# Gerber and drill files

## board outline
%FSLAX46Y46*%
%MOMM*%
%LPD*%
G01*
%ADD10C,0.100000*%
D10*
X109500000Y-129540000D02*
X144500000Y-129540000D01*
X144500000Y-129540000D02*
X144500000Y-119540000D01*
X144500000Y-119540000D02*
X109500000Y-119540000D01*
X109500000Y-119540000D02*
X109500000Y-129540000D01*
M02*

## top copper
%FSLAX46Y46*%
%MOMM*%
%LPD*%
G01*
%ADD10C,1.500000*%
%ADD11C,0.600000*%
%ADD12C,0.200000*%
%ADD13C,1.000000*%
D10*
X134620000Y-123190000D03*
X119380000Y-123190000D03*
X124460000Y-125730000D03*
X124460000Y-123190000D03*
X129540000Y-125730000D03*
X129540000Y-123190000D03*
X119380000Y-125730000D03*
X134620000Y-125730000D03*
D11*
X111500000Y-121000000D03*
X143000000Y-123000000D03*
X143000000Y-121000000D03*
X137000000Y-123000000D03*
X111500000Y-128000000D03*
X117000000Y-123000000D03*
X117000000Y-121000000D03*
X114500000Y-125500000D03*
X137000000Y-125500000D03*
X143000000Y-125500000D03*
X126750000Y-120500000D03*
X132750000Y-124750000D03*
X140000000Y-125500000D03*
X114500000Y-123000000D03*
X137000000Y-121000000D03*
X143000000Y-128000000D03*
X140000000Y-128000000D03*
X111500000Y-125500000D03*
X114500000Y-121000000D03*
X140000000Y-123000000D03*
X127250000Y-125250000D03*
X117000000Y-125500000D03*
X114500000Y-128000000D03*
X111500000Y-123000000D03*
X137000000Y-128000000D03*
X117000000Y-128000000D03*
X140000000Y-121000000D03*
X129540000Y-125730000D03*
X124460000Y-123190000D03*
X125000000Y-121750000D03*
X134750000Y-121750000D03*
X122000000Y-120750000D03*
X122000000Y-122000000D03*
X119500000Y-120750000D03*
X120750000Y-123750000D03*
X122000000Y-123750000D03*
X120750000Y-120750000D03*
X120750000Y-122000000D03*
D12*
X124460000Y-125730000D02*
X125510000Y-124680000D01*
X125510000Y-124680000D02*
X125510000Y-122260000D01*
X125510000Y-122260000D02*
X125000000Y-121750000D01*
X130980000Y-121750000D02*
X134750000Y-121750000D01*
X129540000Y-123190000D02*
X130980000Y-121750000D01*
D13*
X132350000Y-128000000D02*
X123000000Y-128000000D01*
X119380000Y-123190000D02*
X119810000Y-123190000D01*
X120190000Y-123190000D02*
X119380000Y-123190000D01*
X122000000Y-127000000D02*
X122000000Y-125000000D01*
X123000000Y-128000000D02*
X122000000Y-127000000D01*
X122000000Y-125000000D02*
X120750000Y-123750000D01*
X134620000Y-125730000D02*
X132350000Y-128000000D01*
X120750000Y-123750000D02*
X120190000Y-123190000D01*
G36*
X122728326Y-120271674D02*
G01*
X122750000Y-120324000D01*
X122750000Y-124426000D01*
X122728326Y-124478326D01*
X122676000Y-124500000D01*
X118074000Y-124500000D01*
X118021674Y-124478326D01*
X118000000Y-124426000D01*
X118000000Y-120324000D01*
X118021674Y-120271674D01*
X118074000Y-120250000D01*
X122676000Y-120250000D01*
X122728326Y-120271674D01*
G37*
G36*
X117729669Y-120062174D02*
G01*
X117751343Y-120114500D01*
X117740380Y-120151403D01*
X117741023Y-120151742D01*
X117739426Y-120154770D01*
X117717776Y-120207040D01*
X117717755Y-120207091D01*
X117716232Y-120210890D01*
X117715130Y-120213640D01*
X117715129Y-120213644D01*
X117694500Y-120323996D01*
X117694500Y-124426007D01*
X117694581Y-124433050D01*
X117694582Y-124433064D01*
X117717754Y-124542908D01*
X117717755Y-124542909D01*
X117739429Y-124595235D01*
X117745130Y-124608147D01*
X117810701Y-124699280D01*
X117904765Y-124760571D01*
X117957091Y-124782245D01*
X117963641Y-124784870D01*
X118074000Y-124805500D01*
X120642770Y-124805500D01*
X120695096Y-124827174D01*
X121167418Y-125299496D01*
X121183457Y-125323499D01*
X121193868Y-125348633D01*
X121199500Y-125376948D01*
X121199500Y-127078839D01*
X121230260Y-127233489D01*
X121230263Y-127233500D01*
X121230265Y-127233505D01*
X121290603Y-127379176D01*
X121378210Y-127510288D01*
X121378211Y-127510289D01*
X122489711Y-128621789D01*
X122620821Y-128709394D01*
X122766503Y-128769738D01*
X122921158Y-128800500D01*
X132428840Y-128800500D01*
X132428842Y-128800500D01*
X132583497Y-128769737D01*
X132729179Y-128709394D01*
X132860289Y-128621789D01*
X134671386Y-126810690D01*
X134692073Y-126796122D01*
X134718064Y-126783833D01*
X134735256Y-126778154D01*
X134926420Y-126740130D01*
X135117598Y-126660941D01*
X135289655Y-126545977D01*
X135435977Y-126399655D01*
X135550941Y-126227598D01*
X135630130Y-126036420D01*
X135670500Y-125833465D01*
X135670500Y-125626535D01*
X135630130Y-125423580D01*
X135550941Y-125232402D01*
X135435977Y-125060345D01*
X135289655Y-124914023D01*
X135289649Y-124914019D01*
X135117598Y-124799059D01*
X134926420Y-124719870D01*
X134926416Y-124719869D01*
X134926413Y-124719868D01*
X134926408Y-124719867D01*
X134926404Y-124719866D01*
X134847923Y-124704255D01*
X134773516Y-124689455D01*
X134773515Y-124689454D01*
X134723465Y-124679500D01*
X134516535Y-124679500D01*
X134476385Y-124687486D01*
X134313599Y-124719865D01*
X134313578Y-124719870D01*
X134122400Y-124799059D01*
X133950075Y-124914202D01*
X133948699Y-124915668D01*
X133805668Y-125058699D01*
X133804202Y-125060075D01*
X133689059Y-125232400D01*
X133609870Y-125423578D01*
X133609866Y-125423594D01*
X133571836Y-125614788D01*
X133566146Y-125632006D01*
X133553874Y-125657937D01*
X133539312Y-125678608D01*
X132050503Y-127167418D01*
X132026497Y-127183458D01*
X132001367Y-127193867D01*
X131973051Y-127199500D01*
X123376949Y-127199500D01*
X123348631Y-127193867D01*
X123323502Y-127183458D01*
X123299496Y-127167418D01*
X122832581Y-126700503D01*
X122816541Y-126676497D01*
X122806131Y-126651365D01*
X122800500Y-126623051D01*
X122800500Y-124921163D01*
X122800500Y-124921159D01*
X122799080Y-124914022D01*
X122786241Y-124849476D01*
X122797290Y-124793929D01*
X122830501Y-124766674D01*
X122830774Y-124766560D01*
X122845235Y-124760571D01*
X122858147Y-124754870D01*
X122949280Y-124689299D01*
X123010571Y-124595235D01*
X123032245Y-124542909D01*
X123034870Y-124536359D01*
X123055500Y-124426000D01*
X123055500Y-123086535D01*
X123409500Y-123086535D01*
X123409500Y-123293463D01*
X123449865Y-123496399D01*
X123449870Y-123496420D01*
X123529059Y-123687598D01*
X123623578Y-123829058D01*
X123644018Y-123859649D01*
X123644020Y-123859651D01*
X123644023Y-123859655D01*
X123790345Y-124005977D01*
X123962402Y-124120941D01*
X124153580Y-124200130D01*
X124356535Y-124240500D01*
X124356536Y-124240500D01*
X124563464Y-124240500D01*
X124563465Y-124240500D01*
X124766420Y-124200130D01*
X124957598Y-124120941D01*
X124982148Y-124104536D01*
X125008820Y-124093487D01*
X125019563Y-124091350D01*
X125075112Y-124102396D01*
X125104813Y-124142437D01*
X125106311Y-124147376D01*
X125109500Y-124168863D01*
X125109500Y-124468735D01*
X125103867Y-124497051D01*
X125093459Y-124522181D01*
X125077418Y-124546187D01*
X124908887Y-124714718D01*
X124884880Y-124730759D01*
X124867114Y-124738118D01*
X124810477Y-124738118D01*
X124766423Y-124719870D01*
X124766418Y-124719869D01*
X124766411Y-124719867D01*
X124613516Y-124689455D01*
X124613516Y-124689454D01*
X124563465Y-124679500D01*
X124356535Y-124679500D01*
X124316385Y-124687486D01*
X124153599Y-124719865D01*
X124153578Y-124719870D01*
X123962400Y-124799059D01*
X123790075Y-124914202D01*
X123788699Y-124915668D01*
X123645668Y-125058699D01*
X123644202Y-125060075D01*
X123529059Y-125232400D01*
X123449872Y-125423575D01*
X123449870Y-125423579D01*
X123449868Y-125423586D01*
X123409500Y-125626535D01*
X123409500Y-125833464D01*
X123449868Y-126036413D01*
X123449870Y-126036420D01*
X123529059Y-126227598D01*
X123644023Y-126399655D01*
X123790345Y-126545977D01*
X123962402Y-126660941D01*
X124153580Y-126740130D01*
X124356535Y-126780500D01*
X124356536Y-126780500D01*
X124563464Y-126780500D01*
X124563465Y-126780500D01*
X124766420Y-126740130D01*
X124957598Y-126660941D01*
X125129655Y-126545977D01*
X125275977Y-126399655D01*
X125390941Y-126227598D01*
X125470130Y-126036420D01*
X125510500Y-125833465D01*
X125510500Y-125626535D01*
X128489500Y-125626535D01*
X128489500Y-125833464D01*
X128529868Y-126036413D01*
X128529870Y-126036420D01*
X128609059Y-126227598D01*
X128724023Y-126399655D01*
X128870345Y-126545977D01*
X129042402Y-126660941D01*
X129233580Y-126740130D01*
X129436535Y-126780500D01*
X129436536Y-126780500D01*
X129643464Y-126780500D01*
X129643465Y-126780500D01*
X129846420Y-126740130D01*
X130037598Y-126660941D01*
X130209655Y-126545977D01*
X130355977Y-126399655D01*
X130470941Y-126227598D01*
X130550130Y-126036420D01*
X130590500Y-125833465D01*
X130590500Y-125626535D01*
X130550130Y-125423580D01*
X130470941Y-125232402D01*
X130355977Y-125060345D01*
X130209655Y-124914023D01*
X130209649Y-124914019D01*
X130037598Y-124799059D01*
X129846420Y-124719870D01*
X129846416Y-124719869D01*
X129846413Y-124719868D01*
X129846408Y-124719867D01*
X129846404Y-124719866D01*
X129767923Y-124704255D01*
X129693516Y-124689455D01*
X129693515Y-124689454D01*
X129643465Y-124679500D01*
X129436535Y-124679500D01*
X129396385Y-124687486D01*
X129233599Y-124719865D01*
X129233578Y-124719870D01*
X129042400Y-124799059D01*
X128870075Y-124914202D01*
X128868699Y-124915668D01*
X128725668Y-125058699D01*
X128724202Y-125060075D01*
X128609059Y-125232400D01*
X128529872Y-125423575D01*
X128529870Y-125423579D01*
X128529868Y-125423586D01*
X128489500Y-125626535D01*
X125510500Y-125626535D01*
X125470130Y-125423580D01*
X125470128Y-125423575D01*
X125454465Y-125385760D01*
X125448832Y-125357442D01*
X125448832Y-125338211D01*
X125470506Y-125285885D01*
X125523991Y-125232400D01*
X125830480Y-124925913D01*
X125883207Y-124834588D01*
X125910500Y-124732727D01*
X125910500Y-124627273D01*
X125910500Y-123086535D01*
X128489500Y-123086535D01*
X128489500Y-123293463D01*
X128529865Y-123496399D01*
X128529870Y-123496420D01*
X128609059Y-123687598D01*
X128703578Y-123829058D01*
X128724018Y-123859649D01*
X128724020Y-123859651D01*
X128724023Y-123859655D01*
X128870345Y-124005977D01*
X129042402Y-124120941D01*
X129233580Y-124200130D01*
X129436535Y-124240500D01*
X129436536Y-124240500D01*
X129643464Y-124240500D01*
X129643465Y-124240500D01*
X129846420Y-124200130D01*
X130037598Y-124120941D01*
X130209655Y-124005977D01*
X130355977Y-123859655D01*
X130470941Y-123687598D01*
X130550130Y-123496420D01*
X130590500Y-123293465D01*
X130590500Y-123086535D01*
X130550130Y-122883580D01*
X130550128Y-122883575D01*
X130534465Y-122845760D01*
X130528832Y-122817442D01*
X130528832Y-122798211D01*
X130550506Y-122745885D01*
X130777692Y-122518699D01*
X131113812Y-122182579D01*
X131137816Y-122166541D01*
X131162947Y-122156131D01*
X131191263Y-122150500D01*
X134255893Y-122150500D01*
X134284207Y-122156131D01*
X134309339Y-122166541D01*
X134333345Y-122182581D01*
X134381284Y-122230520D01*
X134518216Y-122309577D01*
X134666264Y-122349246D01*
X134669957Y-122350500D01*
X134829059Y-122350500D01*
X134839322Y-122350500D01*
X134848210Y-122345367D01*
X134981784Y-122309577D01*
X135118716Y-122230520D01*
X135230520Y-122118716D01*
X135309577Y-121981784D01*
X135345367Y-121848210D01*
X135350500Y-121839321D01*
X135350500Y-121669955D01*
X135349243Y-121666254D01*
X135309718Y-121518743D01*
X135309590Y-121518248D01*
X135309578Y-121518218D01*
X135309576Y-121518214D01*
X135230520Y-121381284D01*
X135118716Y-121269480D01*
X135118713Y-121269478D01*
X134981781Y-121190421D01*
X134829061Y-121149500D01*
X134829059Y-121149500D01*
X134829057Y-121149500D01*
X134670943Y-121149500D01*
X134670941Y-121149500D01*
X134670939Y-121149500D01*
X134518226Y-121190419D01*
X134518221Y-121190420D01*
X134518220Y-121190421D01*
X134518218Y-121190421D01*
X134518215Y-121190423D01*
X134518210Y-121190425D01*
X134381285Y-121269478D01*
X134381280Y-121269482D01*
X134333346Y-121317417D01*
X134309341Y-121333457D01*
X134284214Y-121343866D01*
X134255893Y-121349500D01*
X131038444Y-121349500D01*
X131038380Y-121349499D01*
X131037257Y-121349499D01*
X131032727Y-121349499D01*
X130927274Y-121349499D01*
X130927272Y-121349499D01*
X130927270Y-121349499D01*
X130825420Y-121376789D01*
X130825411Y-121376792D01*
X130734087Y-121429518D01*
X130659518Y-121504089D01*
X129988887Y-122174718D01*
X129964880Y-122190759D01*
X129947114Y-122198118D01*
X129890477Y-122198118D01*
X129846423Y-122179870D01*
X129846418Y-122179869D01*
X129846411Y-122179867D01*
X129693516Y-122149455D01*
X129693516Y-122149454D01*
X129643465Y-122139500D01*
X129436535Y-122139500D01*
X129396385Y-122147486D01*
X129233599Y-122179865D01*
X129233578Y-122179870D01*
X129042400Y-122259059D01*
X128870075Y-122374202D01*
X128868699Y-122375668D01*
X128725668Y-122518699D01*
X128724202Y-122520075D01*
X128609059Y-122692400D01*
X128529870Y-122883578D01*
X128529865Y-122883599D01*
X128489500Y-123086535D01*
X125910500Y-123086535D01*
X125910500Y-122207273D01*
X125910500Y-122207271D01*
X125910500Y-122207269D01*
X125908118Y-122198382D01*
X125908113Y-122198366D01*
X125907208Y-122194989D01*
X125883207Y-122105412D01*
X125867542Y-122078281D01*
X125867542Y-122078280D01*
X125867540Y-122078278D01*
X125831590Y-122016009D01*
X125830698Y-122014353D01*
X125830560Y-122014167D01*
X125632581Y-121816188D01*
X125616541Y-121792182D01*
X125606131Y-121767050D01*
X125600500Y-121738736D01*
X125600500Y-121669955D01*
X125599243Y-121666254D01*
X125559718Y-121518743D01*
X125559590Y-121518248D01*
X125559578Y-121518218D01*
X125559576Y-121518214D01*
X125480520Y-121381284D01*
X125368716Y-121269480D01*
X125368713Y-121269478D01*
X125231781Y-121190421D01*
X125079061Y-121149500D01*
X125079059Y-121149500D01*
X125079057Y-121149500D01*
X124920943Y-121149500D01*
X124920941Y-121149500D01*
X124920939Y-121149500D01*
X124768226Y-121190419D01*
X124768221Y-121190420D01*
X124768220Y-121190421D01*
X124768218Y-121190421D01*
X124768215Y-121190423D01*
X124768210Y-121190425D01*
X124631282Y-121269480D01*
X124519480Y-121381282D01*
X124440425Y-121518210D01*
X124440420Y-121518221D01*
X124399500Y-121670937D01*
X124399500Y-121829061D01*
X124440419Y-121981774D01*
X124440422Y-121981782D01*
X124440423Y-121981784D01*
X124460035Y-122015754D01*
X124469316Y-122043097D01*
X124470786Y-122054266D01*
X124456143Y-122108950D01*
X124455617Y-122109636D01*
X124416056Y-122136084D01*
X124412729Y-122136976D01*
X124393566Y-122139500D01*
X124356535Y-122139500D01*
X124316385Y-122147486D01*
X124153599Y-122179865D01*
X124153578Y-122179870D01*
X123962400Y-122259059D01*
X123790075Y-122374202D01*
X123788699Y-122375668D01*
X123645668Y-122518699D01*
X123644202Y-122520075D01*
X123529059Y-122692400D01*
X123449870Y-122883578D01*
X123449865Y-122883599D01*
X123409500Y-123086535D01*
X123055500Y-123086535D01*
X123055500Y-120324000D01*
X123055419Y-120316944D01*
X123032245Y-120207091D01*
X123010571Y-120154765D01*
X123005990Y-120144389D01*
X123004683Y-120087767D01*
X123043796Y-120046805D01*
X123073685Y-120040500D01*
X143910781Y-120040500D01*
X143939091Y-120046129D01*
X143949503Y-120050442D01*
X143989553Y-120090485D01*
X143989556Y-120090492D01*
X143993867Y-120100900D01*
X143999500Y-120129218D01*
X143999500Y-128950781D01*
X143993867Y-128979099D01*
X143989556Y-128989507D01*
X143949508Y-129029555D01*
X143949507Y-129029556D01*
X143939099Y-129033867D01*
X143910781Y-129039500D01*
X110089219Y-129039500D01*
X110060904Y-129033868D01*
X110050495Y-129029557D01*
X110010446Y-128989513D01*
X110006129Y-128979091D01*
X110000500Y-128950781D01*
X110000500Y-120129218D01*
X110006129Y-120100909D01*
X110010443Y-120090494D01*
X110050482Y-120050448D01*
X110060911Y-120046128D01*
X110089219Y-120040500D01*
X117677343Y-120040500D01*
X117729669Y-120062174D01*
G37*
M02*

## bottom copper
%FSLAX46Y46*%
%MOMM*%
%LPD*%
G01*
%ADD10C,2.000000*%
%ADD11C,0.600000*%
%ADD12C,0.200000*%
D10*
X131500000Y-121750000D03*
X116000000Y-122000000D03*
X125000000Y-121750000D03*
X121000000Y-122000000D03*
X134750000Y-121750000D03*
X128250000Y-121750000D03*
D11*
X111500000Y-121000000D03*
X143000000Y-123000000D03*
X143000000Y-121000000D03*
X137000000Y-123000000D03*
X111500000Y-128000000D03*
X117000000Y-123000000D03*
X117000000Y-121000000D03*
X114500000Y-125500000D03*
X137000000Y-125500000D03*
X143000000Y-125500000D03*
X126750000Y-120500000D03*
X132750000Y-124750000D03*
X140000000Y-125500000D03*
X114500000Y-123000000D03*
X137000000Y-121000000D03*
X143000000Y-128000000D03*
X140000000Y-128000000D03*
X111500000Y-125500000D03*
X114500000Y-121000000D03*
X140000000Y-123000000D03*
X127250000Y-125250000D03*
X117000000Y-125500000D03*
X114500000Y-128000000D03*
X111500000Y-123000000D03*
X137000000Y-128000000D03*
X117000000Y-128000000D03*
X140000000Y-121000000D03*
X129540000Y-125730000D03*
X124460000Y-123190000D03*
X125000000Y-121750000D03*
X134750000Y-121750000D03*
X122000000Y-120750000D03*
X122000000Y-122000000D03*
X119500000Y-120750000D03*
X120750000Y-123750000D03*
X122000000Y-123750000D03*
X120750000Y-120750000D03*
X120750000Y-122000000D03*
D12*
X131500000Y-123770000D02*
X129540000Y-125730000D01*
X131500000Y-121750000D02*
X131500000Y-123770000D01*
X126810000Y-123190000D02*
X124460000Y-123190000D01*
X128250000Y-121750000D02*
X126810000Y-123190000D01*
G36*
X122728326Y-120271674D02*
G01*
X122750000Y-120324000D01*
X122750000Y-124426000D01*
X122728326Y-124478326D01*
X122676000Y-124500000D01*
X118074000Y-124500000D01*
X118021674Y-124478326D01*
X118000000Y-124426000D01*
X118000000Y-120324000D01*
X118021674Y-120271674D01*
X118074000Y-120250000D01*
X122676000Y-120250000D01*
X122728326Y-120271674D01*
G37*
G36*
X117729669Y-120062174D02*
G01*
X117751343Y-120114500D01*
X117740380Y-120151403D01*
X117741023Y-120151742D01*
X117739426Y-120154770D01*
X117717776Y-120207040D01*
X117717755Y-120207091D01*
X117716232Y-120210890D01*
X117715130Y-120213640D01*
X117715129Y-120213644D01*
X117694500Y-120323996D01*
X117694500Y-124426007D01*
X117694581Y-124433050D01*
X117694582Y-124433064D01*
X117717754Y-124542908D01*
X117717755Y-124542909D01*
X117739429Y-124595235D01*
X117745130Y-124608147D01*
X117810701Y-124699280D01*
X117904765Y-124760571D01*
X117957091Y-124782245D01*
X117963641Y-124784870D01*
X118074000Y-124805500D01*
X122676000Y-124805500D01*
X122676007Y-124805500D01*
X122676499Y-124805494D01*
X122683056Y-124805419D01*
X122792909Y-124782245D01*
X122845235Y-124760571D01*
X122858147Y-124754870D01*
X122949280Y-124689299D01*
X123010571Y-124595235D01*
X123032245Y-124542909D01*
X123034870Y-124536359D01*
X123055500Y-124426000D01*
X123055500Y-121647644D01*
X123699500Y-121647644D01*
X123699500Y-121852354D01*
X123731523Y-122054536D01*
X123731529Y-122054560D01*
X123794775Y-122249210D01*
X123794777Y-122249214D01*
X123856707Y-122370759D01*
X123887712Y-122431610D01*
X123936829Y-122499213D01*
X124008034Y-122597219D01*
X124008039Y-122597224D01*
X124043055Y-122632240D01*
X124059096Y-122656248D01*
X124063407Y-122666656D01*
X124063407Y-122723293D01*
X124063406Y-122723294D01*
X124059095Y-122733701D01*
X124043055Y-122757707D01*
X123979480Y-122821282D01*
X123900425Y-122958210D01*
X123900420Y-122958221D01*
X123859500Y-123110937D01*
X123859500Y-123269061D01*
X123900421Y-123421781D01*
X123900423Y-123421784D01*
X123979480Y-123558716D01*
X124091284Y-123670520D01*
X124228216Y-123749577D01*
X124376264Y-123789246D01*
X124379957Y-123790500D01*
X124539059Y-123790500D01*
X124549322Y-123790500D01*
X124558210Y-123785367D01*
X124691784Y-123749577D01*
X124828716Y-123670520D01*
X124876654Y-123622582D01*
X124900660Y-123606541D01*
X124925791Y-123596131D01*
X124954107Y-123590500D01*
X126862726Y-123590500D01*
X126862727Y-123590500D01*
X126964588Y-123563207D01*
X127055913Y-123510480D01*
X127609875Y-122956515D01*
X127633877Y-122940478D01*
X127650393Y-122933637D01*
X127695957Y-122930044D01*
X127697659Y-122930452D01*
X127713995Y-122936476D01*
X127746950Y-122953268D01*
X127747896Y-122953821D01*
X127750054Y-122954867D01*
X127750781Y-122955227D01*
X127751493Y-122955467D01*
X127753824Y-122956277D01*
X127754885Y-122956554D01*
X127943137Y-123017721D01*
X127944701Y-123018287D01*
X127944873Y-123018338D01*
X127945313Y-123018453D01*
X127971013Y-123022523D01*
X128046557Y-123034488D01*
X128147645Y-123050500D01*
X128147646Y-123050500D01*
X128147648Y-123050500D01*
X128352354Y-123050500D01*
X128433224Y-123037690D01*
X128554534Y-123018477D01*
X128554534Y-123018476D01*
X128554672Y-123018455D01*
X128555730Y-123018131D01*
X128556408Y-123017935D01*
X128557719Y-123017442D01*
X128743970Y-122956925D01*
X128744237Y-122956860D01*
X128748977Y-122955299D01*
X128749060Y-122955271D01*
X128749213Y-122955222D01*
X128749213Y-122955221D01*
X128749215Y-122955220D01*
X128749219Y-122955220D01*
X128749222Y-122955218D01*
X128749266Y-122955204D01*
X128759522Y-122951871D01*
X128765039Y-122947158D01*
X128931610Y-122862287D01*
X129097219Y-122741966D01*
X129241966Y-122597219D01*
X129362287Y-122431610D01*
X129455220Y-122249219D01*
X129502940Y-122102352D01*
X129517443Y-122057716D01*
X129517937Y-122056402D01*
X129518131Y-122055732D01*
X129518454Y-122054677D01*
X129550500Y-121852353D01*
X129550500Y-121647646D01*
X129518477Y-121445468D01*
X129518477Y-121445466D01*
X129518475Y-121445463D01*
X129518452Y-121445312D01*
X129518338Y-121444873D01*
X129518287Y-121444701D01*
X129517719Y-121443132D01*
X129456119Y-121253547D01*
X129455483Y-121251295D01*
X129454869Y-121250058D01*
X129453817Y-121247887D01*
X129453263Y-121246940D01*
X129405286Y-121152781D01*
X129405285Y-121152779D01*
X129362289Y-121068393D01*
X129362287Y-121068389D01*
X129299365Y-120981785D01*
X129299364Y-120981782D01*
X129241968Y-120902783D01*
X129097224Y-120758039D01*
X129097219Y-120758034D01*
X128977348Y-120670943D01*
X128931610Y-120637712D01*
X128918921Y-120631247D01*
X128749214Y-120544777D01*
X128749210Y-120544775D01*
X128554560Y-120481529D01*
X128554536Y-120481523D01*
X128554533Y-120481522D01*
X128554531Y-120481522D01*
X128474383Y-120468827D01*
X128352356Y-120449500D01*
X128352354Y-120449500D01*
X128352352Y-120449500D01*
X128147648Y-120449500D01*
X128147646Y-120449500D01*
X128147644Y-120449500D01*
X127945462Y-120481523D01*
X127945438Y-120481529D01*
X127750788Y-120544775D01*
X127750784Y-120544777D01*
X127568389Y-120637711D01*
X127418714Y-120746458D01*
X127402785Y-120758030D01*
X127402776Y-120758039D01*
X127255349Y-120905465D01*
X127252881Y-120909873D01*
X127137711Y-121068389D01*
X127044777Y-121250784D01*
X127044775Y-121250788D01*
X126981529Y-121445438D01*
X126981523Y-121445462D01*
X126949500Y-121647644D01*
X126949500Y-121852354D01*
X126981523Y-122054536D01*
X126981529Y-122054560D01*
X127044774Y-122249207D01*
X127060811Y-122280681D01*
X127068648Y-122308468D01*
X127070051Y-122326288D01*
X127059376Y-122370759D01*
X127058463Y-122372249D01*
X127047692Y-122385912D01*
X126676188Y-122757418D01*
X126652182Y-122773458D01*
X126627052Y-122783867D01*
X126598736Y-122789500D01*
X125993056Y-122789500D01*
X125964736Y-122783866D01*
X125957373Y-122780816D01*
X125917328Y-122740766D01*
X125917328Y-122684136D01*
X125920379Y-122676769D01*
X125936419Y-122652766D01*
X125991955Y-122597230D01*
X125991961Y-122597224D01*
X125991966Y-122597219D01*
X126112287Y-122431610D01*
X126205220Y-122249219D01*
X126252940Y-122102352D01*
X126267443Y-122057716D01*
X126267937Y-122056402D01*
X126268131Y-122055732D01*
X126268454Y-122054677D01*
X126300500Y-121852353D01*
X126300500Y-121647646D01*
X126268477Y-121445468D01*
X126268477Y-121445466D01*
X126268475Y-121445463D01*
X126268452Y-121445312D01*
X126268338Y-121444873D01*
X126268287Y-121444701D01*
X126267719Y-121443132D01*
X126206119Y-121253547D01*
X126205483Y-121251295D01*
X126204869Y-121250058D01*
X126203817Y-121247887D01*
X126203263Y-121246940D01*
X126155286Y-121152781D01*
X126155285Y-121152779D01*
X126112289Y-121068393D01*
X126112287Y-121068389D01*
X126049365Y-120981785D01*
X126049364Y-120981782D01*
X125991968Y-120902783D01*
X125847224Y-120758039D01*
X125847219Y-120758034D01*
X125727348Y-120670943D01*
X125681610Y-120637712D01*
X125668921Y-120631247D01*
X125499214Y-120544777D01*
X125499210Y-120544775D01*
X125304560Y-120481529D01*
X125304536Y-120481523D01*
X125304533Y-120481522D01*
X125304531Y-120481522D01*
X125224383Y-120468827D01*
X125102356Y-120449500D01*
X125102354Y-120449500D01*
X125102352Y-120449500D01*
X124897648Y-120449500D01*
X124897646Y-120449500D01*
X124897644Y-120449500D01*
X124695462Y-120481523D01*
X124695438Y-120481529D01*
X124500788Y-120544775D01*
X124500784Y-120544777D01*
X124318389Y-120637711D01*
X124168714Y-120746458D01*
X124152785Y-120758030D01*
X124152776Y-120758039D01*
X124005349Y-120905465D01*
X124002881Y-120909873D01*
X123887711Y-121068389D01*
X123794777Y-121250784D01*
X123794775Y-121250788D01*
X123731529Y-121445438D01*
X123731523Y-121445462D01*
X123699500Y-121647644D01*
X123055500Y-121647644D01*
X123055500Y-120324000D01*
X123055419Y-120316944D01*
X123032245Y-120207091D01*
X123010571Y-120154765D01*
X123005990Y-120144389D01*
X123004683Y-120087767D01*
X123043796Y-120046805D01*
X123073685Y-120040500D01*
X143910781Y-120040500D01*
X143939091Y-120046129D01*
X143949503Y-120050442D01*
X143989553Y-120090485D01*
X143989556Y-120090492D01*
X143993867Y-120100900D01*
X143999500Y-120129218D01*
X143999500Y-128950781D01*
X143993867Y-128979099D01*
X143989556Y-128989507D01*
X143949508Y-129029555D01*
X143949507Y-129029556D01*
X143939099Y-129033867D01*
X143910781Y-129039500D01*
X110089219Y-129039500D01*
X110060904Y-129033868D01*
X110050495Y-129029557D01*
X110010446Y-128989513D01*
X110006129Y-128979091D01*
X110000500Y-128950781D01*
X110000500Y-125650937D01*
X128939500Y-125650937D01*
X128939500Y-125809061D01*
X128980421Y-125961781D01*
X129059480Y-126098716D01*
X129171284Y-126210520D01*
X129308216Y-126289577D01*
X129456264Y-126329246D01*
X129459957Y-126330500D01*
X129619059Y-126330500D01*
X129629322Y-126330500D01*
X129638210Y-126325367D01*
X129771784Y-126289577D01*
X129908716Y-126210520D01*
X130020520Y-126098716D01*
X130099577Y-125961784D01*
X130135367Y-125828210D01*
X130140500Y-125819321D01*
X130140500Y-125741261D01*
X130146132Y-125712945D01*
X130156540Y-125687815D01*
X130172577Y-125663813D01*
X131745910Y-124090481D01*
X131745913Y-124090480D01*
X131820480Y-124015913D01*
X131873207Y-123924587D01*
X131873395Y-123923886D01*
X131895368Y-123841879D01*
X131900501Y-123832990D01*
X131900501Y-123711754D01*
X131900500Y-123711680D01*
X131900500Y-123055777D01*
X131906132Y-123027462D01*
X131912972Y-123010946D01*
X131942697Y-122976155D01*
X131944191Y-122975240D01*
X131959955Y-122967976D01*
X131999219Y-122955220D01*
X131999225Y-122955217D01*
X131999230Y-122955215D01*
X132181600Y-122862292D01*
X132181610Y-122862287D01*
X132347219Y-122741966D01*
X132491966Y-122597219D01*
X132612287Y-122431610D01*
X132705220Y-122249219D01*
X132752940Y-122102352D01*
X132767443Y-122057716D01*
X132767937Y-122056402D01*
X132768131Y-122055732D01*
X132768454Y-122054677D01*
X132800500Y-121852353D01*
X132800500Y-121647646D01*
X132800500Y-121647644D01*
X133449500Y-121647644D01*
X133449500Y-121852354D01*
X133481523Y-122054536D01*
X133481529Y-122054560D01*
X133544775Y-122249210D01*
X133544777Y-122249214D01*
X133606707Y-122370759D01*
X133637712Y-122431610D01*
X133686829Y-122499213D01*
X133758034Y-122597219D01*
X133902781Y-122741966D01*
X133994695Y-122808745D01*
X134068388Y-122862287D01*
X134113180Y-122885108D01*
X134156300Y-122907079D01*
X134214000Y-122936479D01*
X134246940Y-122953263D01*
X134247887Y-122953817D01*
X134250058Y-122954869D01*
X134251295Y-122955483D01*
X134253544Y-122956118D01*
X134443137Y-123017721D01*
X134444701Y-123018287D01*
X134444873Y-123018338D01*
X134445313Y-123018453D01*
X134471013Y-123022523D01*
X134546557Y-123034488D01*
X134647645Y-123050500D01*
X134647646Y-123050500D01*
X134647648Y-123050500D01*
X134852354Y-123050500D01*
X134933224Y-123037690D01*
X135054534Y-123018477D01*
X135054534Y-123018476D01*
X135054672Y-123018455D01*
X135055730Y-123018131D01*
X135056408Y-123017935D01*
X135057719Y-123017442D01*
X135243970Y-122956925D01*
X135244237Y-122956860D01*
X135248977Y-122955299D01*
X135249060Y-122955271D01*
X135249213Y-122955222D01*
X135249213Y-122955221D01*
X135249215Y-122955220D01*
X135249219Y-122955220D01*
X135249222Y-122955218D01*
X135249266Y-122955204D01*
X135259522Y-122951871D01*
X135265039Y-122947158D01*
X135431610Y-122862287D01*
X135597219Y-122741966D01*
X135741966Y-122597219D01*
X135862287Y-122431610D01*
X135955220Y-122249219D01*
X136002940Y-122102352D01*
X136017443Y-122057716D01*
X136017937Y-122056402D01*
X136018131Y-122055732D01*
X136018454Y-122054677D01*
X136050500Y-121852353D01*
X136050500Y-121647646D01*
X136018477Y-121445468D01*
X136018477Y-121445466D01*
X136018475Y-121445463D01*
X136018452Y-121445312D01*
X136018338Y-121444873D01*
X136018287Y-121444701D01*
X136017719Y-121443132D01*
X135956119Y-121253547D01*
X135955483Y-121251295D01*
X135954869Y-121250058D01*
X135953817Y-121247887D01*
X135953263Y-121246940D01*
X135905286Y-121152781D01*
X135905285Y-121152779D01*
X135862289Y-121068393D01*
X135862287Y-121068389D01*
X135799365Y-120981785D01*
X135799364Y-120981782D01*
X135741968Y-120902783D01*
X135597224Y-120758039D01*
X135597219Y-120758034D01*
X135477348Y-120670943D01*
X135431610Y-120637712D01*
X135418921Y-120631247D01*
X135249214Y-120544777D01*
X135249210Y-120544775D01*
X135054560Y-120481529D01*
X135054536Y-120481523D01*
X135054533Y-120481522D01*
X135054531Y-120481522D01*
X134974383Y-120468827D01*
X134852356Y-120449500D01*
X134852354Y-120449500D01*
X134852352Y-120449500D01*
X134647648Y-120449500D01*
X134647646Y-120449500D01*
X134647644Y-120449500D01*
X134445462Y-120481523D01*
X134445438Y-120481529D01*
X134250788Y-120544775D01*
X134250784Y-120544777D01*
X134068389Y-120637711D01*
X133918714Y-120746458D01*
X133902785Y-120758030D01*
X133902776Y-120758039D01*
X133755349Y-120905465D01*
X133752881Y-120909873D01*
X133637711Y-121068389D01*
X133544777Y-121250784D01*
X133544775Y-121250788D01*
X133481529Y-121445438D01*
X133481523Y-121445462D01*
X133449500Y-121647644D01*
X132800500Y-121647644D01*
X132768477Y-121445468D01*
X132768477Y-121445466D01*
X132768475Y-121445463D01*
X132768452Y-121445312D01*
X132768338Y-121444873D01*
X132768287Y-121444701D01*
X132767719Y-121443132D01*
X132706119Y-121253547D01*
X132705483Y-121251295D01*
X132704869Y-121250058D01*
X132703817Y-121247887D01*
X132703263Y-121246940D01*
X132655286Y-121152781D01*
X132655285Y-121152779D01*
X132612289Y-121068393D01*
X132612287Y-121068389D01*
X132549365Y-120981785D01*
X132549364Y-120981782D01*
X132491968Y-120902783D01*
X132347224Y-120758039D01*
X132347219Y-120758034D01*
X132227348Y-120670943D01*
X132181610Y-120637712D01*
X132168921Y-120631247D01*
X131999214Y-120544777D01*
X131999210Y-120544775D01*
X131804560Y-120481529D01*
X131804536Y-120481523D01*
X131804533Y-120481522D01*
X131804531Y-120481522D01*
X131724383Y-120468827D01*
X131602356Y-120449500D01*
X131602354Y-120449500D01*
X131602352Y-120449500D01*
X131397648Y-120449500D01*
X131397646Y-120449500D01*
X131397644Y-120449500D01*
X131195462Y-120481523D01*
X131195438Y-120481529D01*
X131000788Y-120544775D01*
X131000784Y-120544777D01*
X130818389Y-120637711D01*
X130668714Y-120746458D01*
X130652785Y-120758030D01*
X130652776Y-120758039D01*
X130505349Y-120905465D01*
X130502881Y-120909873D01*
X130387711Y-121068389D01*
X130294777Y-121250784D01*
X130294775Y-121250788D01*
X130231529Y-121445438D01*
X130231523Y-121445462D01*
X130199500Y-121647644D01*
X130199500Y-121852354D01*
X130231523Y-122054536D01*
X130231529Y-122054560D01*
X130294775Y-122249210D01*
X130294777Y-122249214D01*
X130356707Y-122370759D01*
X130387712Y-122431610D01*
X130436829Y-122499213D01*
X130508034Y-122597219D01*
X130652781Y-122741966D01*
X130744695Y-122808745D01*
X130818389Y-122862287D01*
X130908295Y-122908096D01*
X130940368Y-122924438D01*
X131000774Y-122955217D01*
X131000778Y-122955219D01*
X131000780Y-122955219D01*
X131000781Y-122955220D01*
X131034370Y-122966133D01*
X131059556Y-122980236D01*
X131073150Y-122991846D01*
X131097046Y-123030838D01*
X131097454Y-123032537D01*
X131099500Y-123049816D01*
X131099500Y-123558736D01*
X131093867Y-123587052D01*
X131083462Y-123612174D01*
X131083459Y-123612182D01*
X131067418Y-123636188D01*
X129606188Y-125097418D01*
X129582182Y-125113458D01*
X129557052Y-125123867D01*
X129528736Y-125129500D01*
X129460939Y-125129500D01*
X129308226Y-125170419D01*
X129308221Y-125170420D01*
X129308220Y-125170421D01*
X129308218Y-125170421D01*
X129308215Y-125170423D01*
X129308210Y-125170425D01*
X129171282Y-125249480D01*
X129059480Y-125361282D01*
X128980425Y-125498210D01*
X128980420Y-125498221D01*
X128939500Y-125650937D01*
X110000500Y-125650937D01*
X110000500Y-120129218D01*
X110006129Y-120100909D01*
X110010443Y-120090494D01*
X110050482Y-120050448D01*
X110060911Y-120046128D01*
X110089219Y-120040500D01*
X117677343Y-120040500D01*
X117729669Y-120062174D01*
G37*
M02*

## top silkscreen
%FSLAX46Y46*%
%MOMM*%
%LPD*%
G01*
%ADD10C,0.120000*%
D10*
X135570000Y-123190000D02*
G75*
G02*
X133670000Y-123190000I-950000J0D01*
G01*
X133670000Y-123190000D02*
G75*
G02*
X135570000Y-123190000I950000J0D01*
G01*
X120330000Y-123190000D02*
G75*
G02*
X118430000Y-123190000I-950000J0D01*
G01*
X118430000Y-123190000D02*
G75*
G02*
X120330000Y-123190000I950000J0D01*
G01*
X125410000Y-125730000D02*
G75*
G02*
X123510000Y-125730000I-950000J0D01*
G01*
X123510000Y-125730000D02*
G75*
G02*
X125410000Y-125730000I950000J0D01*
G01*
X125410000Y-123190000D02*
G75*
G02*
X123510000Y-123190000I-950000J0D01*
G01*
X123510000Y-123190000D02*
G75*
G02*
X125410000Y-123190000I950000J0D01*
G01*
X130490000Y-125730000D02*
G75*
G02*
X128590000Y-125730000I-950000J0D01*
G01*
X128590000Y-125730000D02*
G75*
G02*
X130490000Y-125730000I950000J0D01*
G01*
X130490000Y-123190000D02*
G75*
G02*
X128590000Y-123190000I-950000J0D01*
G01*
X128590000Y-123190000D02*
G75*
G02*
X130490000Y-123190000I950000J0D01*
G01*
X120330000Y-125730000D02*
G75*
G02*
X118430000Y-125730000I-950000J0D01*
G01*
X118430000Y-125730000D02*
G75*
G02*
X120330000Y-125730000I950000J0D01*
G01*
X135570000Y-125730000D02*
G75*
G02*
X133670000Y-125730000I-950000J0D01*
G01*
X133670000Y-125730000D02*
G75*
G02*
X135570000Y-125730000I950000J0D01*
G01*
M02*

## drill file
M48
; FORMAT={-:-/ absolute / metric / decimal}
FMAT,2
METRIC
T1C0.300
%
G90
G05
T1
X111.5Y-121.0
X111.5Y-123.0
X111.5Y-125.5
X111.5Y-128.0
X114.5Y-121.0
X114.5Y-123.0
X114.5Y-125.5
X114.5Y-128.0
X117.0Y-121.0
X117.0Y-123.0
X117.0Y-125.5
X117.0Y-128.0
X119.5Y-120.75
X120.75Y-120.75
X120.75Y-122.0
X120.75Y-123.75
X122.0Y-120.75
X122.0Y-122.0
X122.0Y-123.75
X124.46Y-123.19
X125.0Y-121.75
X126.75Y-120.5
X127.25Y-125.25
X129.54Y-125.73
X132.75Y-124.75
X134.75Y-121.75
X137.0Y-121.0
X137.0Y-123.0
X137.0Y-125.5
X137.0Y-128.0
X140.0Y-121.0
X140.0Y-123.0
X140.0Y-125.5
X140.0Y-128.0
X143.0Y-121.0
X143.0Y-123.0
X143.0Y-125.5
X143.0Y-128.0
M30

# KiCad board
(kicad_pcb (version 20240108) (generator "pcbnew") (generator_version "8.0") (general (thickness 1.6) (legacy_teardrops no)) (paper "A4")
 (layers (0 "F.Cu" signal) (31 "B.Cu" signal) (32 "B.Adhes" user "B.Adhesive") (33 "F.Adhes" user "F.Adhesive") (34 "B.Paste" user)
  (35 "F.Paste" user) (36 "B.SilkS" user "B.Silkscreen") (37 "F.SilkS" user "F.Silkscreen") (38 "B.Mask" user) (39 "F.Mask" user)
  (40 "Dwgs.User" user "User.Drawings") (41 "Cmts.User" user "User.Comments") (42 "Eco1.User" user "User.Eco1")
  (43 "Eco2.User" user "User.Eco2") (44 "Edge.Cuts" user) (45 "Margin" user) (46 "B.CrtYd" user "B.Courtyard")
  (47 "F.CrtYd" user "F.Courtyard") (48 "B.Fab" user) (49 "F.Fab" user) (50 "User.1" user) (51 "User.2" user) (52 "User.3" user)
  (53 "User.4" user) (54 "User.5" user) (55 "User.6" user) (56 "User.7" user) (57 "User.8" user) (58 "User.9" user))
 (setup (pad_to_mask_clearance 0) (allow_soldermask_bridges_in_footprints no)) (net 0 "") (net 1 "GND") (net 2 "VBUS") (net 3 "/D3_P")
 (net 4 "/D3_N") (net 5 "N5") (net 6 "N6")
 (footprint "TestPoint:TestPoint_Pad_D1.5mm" (layer "F.Cu") (at 134.62 123.19)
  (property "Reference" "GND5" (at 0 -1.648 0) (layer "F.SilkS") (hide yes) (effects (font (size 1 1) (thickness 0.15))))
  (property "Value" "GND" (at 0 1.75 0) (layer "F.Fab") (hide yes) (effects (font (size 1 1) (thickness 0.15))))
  (fp_circle (center 0 0) (end 0 0.95) (stroke (width 0.12) (type solid)) (fill none) (layer "F.SilkS"))
  (pad "1" smd circle (at 0 0) (size 1.5 1.5) (layers "F.Cu" "F.Mask") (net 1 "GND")))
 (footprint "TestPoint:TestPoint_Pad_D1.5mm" (layer "F.Cu") (at 119.38 123.19)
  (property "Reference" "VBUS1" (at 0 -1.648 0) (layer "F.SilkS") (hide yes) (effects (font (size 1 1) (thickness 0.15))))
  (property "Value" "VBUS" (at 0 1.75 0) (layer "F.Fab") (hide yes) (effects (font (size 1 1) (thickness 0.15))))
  (fp_circle (center 0 0) (end 0 0.95) (stroke (width 0.12) (type solid)) (fill none) (layer "F.SilkS"))
  (pad "1" smd circle (at 0 0) (size 1.5 1.5) (layers "F.Cu" "F.Mask") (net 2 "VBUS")))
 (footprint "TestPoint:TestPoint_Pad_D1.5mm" (layer "F.Cu") (at 124.46 125.73 180)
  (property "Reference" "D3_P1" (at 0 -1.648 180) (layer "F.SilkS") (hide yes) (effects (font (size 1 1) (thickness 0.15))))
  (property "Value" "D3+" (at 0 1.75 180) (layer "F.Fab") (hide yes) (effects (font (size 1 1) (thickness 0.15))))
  (fp_circle (center 0 0) (end 0 0.95) (stroke (width 0.12) (type solid)) (fill none) (layer "F.SilkS"))
  (pad "1" smd circle (at 0 0 180) (size 1.5 1.5) (layers "F.Cu" "F.Mask") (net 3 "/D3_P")))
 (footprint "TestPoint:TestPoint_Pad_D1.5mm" (layer "F.Cu") (at 124.46 123.19)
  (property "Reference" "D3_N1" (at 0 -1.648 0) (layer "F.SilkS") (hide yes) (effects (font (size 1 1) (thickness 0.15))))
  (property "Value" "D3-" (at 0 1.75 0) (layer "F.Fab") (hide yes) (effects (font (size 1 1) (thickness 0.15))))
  (fp_circle (center 0 0) (end 0 0.95) (stroke (width 0.12) (type solid)) (fill none) (layer "F.SilkS"))
  (pad "1" smd circle (at 0 0) (size 1.5 1.5) (layers "F.Cu" "F.Mask") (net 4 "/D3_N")))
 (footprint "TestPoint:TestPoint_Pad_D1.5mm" (layer "F.Cu") (at 129.54 125.73 180)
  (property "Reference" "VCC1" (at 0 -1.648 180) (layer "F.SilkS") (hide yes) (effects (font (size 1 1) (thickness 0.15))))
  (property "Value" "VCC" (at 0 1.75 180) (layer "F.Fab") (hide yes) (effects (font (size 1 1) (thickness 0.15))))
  (fp_circle (center 0 0) (end 0 0.95) (stroke (width 0.12) (type solid)) (fill none) (layer "F.SilkS"))
  (pad "1" smd circle (at 0 0 180) (size 1.5 1.5) (layers "F.Cu" "F.Mask") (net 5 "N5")))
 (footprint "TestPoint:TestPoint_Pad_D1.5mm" (layer "F.Cu") (at 129.54 123.19)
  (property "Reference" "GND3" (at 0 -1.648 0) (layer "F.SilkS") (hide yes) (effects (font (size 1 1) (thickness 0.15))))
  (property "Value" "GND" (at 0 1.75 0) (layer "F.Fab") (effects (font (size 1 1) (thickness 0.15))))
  (fp_circle (center 0 0) (end 0 0.95) (stroke (width 0.12) (type solid)) (fill none) (layer "F.SilkS"))
  (pad "1" smd circle (at 0 0) (size 1.5 1.5) (layers "F.Cu" "F.Mask") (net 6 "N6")))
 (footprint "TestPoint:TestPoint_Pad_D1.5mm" (layer "F.Cu") (at 119.38 125.73 90)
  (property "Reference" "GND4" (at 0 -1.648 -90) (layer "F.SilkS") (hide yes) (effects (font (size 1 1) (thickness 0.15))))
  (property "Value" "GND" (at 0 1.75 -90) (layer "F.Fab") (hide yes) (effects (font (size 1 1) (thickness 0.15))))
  (fp_circle (center 0 0) (end 0 0.95) (stroke (width 0.12) (type solid)) (fill none) (layer "F.SilkS"))
  (pad "1" smd circle (at 0 0 90) (size 1.5 1.5) (layers "F.Cu" "F.Mask") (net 1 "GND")))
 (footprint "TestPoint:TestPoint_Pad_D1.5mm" (layer "F.Cu") (at 134.62 125.73)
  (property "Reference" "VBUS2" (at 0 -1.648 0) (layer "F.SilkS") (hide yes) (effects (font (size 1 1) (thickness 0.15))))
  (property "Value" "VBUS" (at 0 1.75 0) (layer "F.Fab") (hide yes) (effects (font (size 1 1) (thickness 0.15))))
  (fp_circle (center 0 0) (end 0 0.95) (stroke (width 0.12) (type solid)) (fill none) (layer "F.SilkS"))
  (pad "1" smd circle (at 0 0) (size 1.5 1.5) (layers "F.Cu" "F.Mask") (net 2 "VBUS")))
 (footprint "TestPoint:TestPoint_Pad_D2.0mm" (layer "B.Cu") (at 131.5 121.75 180)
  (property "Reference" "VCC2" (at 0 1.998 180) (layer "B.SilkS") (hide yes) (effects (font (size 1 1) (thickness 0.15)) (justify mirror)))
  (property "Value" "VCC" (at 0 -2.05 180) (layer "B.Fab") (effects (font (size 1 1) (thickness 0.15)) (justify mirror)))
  (pad "1" smd circle (at 0 0 180) (size 2 2) (layers "B.Cu" "B.Mask") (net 5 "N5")))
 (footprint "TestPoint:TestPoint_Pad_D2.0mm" (layer "B.Cu") (at 116 122 180)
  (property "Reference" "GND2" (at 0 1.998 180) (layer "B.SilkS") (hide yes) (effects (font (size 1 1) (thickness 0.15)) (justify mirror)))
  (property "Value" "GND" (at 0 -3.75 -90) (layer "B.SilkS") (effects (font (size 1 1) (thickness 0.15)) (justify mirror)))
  (pad "1" smd circle (at 0 0 180) (size 2 2) (layers "B.Cu" "B.Mask") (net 1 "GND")))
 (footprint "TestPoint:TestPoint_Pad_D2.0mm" (layer "B.Cu") (at 125 121.75 180)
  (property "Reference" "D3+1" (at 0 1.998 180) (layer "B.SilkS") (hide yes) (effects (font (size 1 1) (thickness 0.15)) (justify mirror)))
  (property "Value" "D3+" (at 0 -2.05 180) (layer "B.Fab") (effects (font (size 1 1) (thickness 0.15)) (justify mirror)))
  (pad "1" smd circle (at 0 0 180) (size 2 2) (layers "B.Cu" "B.Mask") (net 3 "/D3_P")))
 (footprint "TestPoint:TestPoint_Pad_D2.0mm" (layer "B.Cu") (at 121 122 -90)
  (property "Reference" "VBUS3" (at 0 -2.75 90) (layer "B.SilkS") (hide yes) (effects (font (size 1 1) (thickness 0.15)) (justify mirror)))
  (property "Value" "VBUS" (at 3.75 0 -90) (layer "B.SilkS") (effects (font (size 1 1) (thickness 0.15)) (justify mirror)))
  (pad "1" smd circle (at 0 0 270) (size 2 2) (layers "B.Cu" "B.Mask") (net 2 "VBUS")))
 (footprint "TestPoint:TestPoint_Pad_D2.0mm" (layer "B.Cu") (at 134.75 121.75 180)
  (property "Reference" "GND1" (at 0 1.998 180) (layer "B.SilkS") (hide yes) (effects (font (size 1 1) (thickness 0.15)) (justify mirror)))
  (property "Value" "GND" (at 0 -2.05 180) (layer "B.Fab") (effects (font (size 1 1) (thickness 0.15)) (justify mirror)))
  (pad "1" smd circle (at 0 0 180) (size 2 2) (layers "B.Cu" "B.Mask") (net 6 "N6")))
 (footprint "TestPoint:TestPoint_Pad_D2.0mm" (layer "B.Cu") (at 128.25 121.75 180)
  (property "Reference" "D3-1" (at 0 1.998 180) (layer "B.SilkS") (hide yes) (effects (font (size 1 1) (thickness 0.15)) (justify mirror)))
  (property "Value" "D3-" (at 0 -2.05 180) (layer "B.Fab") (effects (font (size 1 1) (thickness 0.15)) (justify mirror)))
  (pad "1" smd circle (at 0 0 180) (size 2 2) (layers "B.Cu" "B.Mask") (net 4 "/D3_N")))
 (gr_line (start 109.5 129.54) (end 144.5 129.54) (stroke (width 0.1) (type default)) (layer "Edge.Cuts"))
 (gr_line (start 144.5 129.54) (end 144.5 119.54) (stroke (width 0.1) (type default)) (layer "Edge.Cuts"))
 (gr_line (start 144.5 119.54) (end 109.5 119.54) (stroke (width 0.1) (type default)) (layer "Edge.Cuts"))
 (gr_line (start 109.5 119.54) (end 109.5 129.54) (stroke (width 0.1) (type default)) (layer "Edge.Cuts"))
 (via (at 111.5 121) (size 0.6) (drill 0.3) (layers "F.Cu" "B.Cu") (free yes) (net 1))
 (via (at 143 123) (size 0.6) (drill 0.3) (layers "F.Cu" "B.Cu") (free yes) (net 1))
 (via (at 143 121) (size 0.6) (drill 0.3) (layers "F.Cu" "B.Cu") (free yes) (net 1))
 (via (at 137 123) (size 0.6) (drill 0.3) (layers "F.Cu" "B.Cu") (free yes) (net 1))
 (via (at 111.5 128) (size 0.6) (drill 0.3) (layers "F.Cu" "B.Cu") (free yes) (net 1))
 (via (at 117 123) (size 0.6) (drill 0.3) (layers "F.Cu" "B.Cu") (free yes) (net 1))
 (via (at 117 121) (size 0.6) (drill 0.3) (layers "F.Cu" "B.Cu") (free yes) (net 1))
 (via (at 114.5 125.5) (size 0.6) (drill 0.3) (layers "F.Cu" "B.Cu") (free yes) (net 1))
 (via (at 137 125.5) (size 0.6) (drill 0.3) (layers "F.Cu" "B.Cu") (free yes) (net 1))
 (via (at 143 125.5) (size 0.6) (drill 0.3) (layers "F.Cu" "B.Cu") (free yes) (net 1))
 (via (at 126.75 120.5) (size 0.6) (drill 0.3) (layers "F.Cu" "B.Cu") (free yes) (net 1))
 (via (at 132.75 124.75) (size 0.6) (drill 0.3) (layers "F.Cu" "B.Cu") (free yes) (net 1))
 (via (at 140 125.5) (size 0.6) (drill 0.3) (layers "F.Cu" "B.Cu") (free yes) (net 1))
 (via (at 114.5 123) (size 0.6) (drill 0.3) (layers "F.Cu" "B.Cu") (free yes) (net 1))
 (via (at 137 121) (size 0.6) (drill 0.3) (layers "F.Cu" "B.Cu") (free yes) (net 1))
 (via (at 143 128) (size 0.6) (drill 0.3) (layers "F.Cu" "B.Cu") (free yes) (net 1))
 (via (at 140 128) (size 0.6) (drill 0.3) (layers "F.Cu" "B.Cu") (free yes) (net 1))
 (via (at 111.5 125.5) (size 0.6) (drill 0.3) (layers "F.Cu" "B.Cu") (free yes) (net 1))
 (via (at 114.5 121) (size 0.6) (drill 0.3) (layers "F.Cu" "B.Cu") (free yes) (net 1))
 (via (at 140 123) (size 0.6) (drill 0.3) (layers "F.Cu" "B.Cu") (free yes) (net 1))
 (via (at 127.25 125.25) (size 0.6) (drill 0.3) (layers "F.Cu" "B.Cu") (free yes) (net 1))
 (via (at 117 125.5) (size 0.6) (drill 0.3) (layers "F.Cu" "B.Cu") (free yes) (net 1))
 (via (at 114.5 128) (size 0.6) (drill 0.3) (layers "F.Cu" "B.Cu") (free yes) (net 1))
 (via (at 111.5 123) (size 0.6) (drill 0.3) (layers "F.Cu" "B.Cu") (free yes) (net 1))
 (via (at 137 128) (size 0.6) (drill 0.3) (layers "F.Cu" "B.Cu") (free yes) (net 1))
 (via (at 117 128) (size 0.6) (drill 0.3) (layers "F.Cu" "B.Cu") (free yes) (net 1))
 (via (at 140 121) (size 0.6) (drill 0.3) (layers "F.Cu" "B.Cu") (free yes) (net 1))
 (via (at 129.54 125.73) (size 0.6) (drill 0.3) (layers "F.Cu" "B.Cu") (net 5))
 (segment (start 131.5 123.77) (end 129.54 125.73) (width 0.2) (layer "B.Cu") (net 5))
 (segment (start 131.5 121.75) (end 131.5 123.77) (width 0.2) (layer "B.Cu") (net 5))
 (via (at 124.46 123.19) (size 0.6) (drill 0.3) (layers "F.Cu" "B.Cu") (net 4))
 (segment (start 126.81 123.19) (end 124.46 123.19) (width 0.2) (layer "B.Cu") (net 4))
 (segment (start 128.25 121.75) (end 126.81 123.19) (width 0.2) (layer "B.Cu") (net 4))
 (segment (start 124.46 125.73) (end 125.51 124.68) (width 0.2) (layer "F.Cu") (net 3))
 (segment (start 125.51 124.68) (end 125.51 122.26) (width 0.2) (layer "F.Cu") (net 3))
 (segment (start 125.51 122.26) (end 125 121.75) (width 0.2) (layer "F.Cu") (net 3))
 (via (at 125 121.75) (size 0.6) (drill 0.3) (layers "F.Cu" "B.Cu") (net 3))
 (segment (start 130.98 121.75) (end 134.75 121.75) (width 0.2) (layer "F.Cu") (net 6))
 (segment (start 129.54 123.19) (end 130.98 121.75) (width 0.2) (layer "F.Cu") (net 6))
 (via (at 134.75 121.75) (size 0.6) (drill 0.3) (layers "F.Cu" "B.Cu") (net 6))
 (segment (start 132.35 128) (end 123 128) (width 1) (layer "F.Cu") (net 2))
 (segment (start 119.38 123.19) (end 119.81 123.19) (width 1) (layer "F.Cu") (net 2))
 (segment (start 120.19 123.19) (end 119.38 123.19) (width 1) (layer "F.Cu") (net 2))
 (segment (start 122 127) (end 122 125) (width 1) (layer "F.Cu") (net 2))
 (segment (start 123 128) (end 122 127) (width 1) (layer "F.Cu") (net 2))
 (segment (start 122 125) (end 120.75 123.75) (width 1) (layer "F.Cu") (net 2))
 (segment (start 134.62 125.73) (end 132.35 128) (width 1) (layer "F.Cu") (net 2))
 (segment (start 120.75 123.75) (end 120.19 123.19) (width 1) (layer "F.Cu") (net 2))
 (via (at 122 120.75) (size 0.6) (drill 0.3) (layers "F.Cu" "B.Cu") (free yes) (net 2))
 (via (at 122 122) (size 0.6) (drill 0.3) (layers "F.Cu" "B.Cu") (free yes) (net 2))
 (via (at 119.5 120.75) (size 0.6) (drill 0.3) (layers "F.Cu" "B.Cu") (free yes) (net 2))
 (via (at 120.75 123.75) (size 0.6) (drill 0.3) (layers "F.Cu" "B.Cu") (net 2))
 (via (at 122 123.75) (size 0.6) (drill 0.3) (layers "F.Cu" "B.Cu") (free yes) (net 2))
 (via (at 120.75 120.75) (size 0.6) (drill 0.3) (layers "F.Cu" "B.Cu") (free yes) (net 2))
 (via (at 120.75 122) (size 0.6) (drill 0.3) (layers "F.Cu" "B.Cu") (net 2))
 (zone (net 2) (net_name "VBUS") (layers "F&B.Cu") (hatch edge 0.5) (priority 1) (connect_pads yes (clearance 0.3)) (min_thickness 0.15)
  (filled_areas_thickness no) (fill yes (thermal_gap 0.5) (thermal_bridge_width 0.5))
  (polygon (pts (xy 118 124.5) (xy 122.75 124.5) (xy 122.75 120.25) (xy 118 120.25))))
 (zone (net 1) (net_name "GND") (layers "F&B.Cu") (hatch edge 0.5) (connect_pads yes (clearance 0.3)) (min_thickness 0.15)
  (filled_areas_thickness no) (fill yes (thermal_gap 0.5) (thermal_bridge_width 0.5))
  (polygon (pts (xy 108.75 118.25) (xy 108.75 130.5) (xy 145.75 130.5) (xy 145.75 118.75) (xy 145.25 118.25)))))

